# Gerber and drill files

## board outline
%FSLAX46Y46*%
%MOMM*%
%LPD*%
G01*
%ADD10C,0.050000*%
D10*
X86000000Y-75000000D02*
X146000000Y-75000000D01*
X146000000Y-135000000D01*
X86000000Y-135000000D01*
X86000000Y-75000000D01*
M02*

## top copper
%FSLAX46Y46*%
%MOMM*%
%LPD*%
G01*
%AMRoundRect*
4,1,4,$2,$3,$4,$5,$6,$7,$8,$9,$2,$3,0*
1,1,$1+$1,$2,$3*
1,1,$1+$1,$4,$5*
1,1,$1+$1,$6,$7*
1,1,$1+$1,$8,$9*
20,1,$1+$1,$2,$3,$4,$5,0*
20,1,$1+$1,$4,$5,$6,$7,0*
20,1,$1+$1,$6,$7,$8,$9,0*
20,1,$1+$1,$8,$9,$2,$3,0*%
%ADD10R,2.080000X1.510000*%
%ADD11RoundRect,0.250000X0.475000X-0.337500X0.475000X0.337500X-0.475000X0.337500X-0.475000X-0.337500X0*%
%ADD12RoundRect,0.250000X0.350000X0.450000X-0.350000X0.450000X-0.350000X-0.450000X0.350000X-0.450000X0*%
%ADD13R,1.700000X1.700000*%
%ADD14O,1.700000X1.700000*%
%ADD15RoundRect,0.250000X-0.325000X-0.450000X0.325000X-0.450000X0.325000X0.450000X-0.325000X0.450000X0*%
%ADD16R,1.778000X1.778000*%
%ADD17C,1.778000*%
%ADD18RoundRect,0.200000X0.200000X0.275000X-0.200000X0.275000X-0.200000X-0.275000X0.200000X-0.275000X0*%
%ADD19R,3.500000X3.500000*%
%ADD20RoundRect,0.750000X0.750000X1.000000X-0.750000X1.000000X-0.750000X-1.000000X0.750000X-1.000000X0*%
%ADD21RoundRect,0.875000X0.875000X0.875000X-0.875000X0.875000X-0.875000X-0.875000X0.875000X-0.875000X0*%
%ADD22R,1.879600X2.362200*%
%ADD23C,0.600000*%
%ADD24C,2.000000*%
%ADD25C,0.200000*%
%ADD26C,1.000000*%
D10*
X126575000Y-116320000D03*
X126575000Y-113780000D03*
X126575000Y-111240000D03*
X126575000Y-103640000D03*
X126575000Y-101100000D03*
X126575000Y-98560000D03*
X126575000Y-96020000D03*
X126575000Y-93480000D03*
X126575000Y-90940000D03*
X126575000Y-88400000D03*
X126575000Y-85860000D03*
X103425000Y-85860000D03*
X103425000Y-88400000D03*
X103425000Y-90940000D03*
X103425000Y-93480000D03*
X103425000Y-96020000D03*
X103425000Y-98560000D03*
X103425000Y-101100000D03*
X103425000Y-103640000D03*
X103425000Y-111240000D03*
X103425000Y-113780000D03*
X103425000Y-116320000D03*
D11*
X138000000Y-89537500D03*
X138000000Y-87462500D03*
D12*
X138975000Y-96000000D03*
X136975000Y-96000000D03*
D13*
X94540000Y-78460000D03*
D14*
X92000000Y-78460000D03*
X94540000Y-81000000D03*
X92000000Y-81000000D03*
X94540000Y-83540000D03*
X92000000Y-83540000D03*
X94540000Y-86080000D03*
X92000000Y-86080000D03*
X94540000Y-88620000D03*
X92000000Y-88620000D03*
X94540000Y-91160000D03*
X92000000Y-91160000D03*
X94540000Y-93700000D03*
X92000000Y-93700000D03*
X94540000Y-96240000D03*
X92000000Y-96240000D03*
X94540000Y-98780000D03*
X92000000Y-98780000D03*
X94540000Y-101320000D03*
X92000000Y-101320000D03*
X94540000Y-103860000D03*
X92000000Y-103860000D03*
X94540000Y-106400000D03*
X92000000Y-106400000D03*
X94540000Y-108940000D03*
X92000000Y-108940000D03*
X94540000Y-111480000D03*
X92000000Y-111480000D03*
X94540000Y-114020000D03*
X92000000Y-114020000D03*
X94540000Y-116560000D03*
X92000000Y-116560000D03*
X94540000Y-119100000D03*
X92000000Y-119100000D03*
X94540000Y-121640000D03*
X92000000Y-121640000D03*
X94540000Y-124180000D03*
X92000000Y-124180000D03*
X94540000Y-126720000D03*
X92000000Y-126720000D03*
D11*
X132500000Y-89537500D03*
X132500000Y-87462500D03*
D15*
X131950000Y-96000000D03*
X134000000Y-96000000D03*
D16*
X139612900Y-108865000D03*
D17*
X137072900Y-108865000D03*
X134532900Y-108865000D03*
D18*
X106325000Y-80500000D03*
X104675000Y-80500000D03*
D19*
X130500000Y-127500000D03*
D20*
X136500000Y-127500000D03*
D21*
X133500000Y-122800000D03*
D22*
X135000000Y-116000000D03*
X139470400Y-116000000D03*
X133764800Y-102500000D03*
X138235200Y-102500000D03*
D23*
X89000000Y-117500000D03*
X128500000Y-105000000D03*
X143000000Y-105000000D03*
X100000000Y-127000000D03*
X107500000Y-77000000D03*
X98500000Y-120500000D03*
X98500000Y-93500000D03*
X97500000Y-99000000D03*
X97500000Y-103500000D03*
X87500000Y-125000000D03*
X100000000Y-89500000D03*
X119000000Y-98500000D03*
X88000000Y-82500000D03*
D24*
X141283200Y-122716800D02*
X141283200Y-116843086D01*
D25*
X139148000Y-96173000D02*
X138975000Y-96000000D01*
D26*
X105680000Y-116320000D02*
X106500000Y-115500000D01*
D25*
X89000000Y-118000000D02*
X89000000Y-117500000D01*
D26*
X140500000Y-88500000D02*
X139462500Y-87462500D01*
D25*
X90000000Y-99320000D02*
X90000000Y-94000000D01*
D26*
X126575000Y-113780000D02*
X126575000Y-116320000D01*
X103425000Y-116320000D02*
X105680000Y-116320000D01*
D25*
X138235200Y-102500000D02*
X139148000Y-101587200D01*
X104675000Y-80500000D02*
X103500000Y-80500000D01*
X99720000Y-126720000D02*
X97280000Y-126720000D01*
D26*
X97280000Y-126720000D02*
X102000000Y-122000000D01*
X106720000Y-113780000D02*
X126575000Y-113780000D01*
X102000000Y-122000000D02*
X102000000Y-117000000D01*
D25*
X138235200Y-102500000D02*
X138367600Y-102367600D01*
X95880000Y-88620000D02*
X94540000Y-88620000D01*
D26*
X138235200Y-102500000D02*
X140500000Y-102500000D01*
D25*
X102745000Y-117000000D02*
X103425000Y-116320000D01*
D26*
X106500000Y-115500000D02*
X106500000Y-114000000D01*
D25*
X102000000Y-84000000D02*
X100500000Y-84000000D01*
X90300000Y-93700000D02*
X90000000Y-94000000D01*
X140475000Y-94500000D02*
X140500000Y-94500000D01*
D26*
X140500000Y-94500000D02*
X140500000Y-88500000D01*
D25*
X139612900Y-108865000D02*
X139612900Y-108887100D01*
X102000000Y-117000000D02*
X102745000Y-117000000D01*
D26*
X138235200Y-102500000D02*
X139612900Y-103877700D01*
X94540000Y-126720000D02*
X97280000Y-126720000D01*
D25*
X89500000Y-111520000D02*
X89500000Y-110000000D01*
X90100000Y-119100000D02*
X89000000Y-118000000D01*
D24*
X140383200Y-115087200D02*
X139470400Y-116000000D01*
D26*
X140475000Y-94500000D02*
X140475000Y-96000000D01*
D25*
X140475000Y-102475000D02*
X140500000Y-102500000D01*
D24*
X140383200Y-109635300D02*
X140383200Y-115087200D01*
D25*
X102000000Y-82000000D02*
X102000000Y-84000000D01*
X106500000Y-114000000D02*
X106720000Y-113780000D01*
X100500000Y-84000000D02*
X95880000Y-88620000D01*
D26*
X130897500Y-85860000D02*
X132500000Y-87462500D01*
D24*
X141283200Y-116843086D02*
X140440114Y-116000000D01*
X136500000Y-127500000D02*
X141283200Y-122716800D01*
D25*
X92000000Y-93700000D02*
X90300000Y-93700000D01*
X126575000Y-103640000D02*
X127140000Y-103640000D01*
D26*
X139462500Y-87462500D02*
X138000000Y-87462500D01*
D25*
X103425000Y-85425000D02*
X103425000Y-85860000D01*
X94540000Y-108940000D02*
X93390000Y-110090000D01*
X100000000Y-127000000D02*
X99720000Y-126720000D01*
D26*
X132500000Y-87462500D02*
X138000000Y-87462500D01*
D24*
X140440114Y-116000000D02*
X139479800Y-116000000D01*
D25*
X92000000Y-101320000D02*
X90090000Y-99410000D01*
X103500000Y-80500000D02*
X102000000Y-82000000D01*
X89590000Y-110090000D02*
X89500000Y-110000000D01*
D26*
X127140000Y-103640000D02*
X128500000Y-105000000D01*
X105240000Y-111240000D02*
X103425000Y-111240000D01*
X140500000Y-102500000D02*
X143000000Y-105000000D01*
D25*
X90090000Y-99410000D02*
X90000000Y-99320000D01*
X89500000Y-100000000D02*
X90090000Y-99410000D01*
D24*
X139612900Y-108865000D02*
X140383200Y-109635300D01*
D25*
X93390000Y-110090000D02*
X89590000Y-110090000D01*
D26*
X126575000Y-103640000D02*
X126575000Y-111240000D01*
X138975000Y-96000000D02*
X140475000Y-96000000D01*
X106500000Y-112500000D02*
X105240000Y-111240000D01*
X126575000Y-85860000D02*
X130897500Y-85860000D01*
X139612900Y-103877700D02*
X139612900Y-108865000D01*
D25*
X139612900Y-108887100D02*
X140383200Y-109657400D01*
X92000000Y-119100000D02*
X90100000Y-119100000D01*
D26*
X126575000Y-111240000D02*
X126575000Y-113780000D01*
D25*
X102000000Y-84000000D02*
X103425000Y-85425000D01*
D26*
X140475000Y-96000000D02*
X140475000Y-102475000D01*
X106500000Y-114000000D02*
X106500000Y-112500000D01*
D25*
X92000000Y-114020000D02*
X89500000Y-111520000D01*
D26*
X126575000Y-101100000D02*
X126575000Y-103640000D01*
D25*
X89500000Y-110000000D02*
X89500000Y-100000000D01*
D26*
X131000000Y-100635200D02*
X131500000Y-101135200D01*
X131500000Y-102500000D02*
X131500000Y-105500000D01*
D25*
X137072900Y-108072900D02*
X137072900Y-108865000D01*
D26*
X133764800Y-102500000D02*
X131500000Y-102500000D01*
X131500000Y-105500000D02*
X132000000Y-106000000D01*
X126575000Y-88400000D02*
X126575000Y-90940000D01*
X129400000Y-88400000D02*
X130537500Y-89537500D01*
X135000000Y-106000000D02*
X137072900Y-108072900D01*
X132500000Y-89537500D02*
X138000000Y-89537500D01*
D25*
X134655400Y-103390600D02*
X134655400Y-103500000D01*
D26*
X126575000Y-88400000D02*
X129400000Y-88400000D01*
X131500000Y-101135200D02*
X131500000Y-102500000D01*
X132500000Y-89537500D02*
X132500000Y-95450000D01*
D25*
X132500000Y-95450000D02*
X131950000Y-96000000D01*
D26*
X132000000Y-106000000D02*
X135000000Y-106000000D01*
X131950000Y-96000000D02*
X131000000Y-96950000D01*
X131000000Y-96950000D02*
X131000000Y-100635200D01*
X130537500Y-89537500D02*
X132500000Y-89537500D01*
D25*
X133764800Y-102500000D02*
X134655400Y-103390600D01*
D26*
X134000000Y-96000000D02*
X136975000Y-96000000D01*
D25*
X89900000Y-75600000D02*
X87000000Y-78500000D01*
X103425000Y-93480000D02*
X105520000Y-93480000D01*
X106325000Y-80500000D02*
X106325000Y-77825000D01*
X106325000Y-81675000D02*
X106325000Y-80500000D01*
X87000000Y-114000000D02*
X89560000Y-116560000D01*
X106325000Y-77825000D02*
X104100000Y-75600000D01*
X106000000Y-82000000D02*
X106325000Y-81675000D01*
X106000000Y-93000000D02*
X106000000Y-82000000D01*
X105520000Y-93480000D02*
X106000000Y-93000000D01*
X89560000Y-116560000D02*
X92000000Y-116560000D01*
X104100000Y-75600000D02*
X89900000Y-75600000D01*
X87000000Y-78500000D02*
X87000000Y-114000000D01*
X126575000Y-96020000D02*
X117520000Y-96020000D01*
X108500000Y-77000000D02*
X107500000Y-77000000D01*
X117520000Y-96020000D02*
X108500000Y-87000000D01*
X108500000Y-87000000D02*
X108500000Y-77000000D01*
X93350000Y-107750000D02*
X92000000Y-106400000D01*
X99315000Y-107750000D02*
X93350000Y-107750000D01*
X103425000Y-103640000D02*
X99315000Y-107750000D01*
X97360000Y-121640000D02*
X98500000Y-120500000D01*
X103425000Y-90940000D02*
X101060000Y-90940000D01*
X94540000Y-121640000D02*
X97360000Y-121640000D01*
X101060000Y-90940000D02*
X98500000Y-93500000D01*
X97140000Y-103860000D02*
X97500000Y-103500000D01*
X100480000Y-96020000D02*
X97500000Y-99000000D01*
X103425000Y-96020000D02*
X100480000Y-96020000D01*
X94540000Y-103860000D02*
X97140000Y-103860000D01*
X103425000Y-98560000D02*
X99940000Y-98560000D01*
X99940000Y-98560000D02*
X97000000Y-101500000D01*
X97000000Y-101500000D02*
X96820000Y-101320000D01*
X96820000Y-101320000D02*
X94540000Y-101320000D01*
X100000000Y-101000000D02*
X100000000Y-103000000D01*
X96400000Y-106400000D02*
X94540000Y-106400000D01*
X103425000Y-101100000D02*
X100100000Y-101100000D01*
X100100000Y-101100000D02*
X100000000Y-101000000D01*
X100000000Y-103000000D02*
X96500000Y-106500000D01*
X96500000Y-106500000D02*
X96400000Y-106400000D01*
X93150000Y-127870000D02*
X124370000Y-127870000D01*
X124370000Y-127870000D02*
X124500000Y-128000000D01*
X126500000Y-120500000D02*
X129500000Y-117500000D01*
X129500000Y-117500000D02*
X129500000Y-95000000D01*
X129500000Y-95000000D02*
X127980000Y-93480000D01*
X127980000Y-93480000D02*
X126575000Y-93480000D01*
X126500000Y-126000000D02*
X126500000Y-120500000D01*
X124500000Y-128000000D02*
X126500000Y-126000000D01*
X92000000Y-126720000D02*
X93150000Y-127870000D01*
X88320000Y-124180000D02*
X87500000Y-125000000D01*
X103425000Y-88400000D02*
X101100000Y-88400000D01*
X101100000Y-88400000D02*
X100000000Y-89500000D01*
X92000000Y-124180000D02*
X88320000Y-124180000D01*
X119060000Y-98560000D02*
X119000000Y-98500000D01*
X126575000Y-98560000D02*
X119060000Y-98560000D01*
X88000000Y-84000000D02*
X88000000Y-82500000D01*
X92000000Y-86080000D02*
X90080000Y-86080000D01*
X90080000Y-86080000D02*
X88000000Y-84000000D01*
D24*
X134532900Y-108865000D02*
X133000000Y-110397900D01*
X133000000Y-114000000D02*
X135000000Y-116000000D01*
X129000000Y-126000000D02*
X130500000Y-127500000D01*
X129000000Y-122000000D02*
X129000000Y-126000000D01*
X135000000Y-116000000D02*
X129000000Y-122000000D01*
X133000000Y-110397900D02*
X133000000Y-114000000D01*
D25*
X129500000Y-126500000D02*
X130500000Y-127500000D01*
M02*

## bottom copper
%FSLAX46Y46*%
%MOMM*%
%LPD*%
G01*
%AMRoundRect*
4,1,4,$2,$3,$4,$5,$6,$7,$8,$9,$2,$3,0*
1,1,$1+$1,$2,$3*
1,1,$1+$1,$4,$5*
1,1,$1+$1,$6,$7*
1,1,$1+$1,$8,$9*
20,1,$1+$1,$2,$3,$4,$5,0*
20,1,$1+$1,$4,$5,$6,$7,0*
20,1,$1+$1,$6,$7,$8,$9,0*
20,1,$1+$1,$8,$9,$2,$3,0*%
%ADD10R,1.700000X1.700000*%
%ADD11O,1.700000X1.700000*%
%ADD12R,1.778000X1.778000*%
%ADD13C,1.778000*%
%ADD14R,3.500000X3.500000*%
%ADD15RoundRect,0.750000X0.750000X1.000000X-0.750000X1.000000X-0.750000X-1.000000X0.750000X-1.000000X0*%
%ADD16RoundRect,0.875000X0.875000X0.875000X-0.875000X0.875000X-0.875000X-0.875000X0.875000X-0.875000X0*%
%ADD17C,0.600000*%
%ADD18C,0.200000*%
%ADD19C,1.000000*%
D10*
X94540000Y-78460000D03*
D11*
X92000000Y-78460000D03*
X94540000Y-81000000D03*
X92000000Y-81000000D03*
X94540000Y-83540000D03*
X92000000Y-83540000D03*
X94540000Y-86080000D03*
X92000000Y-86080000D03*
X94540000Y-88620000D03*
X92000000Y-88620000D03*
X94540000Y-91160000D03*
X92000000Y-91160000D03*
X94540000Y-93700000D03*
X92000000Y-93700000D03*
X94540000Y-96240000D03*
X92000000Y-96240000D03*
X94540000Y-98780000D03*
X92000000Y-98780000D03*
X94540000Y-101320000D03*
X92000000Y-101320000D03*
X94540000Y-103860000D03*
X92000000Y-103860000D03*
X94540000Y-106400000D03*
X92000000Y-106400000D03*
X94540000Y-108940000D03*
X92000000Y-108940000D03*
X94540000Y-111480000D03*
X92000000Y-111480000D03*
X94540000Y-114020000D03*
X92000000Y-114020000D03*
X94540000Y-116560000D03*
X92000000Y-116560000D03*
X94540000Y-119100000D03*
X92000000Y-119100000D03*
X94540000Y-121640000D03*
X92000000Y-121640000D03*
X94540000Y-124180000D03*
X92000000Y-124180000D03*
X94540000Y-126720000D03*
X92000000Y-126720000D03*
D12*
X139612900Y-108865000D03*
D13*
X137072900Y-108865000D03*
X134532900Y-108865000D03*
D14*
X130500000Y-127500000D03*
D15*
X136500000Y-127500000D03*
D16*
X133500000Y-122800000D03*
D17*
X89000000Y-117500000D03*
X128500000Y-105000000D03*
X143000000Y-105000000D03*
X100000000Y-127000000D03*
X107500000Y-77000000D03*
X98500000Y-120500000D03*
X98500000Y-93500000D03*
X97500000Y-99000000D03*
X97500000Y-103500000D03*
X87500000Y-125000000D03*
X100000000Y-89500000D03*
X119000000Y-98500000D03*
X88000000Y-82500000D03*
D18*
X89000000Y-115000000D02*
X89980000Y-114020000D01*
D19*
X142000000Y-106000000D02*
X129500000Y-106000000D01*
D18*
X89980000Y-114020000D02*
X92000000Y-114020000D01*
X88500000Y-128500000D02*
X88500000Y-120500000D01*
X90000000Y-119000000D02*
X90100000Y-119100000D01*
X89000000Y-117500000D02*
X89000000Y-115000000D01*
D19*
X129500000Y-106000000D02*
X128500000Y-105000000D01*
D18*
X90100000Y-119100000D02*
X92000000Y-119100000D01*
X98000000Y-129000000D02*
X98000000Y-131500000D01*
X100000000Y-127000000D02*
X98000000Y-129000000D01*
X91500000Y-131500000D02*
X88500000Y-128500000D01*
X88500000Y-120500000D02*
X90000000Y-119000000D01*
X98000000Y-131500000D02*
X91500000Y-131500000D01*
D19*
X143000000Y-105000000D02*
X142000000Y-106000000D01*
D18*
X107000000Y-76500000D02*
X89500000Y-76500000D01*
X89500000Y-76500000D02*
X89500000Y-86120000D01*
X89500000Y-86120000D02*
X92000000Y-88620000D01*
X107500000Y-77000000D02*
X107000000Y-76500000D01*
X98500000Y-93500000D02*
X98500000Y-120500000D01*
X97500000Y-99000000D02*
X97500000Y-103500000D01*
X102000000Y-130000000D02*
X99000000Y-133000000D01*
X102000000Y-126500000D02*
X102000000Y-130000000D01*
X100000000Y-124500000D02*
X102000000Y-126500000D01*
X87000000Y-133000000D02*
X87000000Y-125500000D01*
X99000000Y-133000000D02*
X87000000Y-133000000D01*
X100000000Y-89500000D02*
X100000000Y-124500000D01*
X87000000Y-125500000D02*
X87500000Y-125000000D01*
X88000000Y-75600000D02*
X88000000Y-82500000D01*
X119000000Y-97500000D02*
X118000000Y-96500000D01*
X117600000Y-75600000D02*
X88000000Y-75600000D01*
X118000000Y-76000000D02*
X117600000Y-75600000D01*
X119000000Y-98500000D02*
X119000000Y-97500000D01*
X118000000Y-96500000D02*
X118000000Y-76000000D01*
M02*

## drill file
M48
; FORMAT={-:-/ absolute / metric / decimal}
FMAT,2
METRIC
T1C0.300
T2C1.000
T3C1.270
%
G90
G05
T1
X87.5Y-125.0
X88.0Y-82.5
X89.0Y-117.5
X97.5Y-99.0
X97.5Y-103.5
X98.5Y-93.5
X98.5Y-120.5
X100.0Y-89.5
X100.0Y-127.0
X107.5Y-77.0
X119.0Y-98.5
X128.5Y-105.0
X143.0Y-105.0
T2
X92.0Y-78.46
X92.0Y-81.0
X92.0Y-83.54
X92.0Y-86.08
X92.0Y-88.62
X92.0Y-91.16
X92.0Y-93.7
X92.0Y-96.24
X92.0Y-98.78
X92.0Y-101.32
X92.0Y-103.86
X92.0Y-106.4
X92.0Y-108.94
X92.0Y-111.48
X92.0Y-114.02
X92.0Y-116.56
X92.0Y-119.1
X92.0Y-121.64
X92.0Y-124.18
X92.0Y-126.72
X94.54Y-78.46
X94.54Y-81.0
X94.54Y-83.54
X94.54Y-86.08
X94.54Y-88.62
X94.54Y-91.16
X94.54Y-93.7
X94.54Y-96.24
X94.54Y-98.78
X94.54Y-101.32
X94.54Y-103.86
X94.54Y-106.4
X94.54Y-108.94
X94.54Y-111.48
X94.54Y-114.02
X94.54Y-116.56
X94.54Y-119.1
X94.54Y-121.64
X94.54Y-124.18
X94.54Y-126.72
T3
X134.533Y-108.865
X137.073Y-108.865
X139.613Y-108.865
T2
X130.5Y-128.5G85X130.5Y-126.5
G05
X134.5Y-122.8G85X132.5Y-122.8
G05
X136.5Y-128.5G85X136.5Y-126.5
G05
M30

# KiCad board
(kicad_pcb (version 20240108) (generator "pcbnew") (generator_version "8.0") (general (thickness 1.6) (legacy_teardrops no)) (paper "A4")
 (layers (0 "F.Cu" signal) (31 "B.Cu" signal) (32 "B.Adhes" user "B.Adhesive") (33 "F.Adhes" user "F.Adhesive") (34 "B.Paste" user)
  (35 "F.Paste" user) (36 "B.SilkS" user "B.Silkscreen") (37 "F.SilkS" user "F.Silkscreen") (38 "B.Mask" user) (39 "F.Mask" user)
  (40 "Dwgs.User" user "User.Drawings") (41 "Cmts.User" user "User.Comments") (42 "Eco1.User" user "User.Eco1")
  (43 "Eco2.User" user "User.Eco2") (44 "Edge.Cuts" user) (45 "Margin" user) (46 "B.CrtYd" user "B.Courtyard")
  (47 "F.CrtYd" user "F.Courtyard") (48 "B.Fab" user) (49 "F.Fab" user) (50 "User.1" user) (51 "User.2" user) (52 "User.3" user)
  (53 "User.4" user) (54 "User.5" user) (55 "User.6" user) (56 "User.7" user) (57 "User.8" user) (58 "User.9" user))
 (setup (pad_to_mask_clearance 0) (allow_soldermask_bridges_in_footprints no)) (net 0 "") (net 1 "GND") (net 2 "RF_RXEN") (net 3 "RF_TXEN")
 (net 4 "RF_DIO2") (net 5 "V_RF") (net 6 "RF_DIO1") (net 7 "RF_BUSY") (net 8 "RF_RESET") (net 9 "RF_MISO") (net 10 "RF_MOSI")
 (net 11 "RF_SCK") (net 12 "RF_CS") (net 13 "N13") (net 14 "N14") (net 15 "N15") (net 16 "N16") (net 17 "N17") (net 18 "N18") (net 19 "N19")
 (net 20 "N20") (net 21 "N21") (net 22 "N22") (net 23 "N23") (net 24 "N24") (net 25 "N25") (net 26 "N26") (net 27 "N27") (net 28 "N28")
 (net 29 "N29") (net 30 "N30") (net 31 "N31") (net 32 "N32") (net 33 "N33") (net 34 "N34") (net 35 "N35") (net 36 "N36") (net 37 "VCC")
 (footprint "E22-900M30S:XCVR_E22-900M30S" (layer "F.Cu") (at 115 102.5)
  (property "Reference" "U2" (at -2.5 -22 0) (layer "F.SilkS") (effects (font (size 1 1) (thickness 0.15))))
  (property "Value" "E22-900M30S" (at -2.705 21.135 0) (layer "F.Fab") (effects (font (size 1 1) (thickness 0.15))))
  (pad "1" smd rect (at 11.575 13.82) (size 2.08 1.51) (layers "F.Cu" "F.Paste" "F.Mask") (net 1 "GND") (solder_mask_margin 0.102))
  (pad "2" smd rect (at 11.575 11.28) (size 2.08 1.51) (layers "F.Cu" "F.Paste" "F.Mask") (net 1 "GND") (solder_mask_margin 0.102))
  (pad "3" smd rect (at 11.575 8.74) (size 2.08 1.51) (layers "F.Cu" "F.Paste" "F.Mask") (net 1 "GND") (solder_mask_margin 0.102))
  (pad "4" smd rect (at 11.575 1.14) (size 2.08 1.51) (layers "F.Cu" "F.Paste" "F.Mask") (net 1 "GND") (solder_mask_margin 0.102))
  (pad "5" smd rect (at 11.575 -1.4) (size 2.08 1.51) (layers "F.Cu" "F.Paste" "F.Mask") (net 1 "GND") (solder_mask_margin 0.102))
  (pad "6" smd rect (at 11.575 -3.94) (size 2.08 1.51) (layers "F.Cu" "F.Paste" "F.Mask") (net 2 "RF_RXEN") (solder_mask_margin 0.102))
  (pad "7" smd rect (at 11.575 -6.48) (size 2.08 1.51) (layers "F.Cu" "F.Paste" "F.Mask") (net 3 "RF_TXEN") (solder_mask_margin 0.102))
  (pad "8" smd rect (at 11.575 -9.02) (size 2.08 1.51) (layers "F.Cu" "F.Paste" "F.Mask") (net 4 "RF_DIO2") (solder_mask_margin 0.102))
  (pad "9" smd rect (at 11.575 -11.56) (size 2.08 1.51) (layers "F.Cu" "F.Paste" "F.Mask") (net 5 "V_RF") (solder_mask_margin 0.102))
  (pad "10" smd rect (at 11.575 -14.1) (size 2.08 1.51) (layers "F.Cu" "F.Paste" "F.Mask") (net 5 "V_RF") (solder_mask_margin 0.102))
  (pad "11" smd rect (at 11.575 -16.64) (size 2.08 1.51) (layers "F.Cu" "F.Paste" "F.Mask") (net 1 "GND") (solder_mask_margin 0.102))
  (pad "12" smd rect (at -11.575 -16.64) (size 2.08 1.51) (layers "F.Cu" "F.Paste" "F.Mask") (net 1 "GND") (solder_mask_margin 0.102))
  (pad "13" smd rect (at -11.575 -14.1) (size 2.08 1.51) (layers "F.Cu" "F.Paste" "F.Mask") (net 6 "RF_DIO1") (solder_mask_margin 0.102))
  (pad "14" smd rect (at -11.575 -11.56) (size 2.08 1.51) (layers "F.Cu" "F.Paste" "F.Mask") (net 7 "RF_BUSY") (solder_mask_margin 0.102))
  (pad "15" smd rect (at -11.575 -9.02) (size 2.08 1.51) (layers "F.Cu" "F.Paste" "F.Mask") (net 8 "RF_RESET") (solder_mask_margin 0.102))
  (pad "16" smd rect (at -11.575 -6.48) (size 2.08 1.51) (layers "F.Cu" "F.Paste" "F.Mask") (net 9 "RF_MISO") (solder_mask_margin 0.102))
  (pad "17" smd rect (at -11.575 -3.94) (size 2.08 1.51) (layers "F.Cu" "F.Paste" "F.Mask") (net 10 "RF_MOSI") (solder_mask_margin 0.102))
  (pad "18" smd rect (at -11.575 -1.4) (size 2.08 1.51) (layers "F.Cu" "F.Paste" "F.Mask") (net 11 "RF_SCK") (solder_mask_margin 0.102))
  (pad "19" smd rect (at -11.575 1.14) (size 2.08 1.51) (layers "F.Cu" "F.Paste" "F.Mask") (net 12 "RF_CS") (solder_mask_margin 0.102))
  (pad "20" smd rect (at -11.575 8.74) (size 2.08 1.51) (layers "F.Cu" "F.Paste" "F.Mask") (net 1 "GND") (solder_mask_margin 0.102))
  (pad "21" smd rect (at -11.575 11.28) (size 2.08 1.51) (layers "F.Cu" "F.Paste" "F.Mask") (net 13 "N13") (solder_mask_margin 0.102))
  (pad "22" smd rect (at -11.575 13.82) (size 2.08 1.51) (layers "F.Cu" "F.Paste" "F.Mask") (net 1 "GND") (solder_mask_margin 0.102)))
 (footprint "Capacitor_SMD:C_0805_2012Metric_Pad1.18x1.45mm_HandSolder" (layer "F.Cu") (at 138 88.5 90)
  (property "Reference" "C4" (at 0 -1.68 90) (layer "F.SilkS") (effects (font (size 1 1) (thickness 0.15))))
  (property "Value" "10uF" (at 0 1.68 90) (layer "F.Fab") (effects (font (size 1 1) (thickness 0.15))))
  (pad "1" smd roundrect (at -1.0375 0 90) (size 1.175 1.45) (layers "F.Cu" "F.Paste" "F.Mask") (roundrect_rratio 0.212766) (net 5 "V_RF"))
  (pad "2" smd roundrect (at 1.0375 0 90) (size 1.175 1.45) (layers "F.Cu" "F.Paste" "F.Mask") (roundrect_rratio 0.212766) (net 1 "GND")))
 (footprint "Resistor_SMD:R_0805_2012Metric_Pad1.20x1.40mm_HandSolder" (layer "F.Cu") (at 137.975 96 180)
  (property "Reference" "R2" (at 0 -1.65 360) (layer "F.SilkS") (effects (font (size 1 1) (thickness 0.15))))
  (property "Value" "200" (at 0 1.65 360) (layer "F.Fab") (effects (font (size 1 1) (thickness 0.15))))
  (pad "1" smd roundrect (at -1 0 180) (size 1.2 1.4) (layers "F.Cu" "F.Paste" "F.Mask") (roundrect_rratio 0.208333) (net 1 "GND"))
  (pad "2" smd roundrect (at 1 0 180) (size 1.2 1.4) (layers "F.Cu" "F.Paste" "F.Mask") (roundrect_rratio 0.208333) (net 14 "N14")))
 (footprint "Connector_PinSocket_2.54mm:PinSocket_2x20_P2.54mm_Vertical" (layer "F.Cu") (at 94.54 78.46)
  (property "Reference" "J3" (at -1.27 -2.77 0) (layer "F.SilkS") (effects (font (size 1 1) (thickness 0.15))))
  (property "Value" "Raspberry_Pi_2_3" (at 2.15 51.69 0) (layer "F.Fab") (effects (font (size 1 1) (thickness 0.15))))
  (pad "1" thru_hole rect (at 0 0) (size 1.7 1.7) (drill 1) (layers "*.Cu" "*.Mask") (remove_unused_layers no) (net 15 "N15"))
  (pad "2" thru_hole oval (at -2.54 0) (size 1.7 1.7) (drill 1) (layers "*.Cu" "*.Mask") (remove_unused_layers no) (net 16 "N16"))
  (pad "3" thru_hole oval (at 0 2.54) (size 1.7 1.7) (drill 1) (layers "*.Cu" "*.Mask") (remove_unused_layers no) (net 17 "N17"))
  (pad "4" thru_hole oval (at -2.54 2.54) (size 1.7 1.7) (drill 1) (layers "*.Cu" "*.Mask") (remove_unused_layers no) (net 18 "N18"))
  (pad "5" thru_hole oval (at 0 5.08) (size 1.7 1.7) (drill 1) (layers "*.Cu" "*.Mask") (remove_unused_layers no) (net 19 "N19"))
  (pad "6" thru_hole oval (at -2.54 5.08) (size 1.7 1.7) (drill 1) (layers "*.Cu" "*.Mask") (remove_unused_layers no) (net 1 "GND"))
  (pad "7" thru_hole oval (at 0 7.62) (size 1.7 1.7) (drill 1) (layers "*.Cu" "*.Mask") (remove_unused_layers no) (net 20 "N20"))
  (pad "8" thru_hole oval (at -2.54 7.62) (size 1.7 1.7) (drill 1) (layers "*.Cu" "*.Mask") (remove_unused_layers no) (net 2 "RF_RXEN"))
  (pad "9" thru_hole oval (at 0 10.16) (size 1.7 1.7) (drill 1) (layers "*.Cu" "*.Mask") (remove_unused_layers no) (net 1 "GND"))
  (pad "10" thru_hole oval (at -2.54 10.16) (size 1.7 1.7) (drill 1) (layers "*.Cu" "*.Mask") (remove_unused_layers no) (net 3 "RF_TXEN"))
  (pad "11" thru_hole oval (at 0 12.7) (size 1.7 1.7) (drill 1) (layers "*.Cu" "*.Mask") (remove_unused_layers no) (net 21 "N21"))
  (pad "12" thru_hole oval (at -2.54 12.7) (size 1.7 1.7) (drill 1) (layers "*.Cu" "*.Mask") (remove_unused_layers no) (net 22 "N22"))
  (pad "13" thru_hole oval (at 0 15.24) (size 1.7 1.7) (drill 1) (layers "*.Cu" "*.Mask") (remove_unused_layers no) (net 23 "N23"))
  (pad "14" thru_hole oval (at -2.54 15.24) (size 1.7 1.7) (drill 1) (layers "*.Cu" "*.Mask") (remove_unused_layers no) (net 1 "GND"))
  (pad "15" thru_hole oval (at 0 17.78) (size 1.7 1.7) (drill 1) (layers "*.Cu" "*.Mask") (remove_unused_layers no) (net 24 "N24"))
  (pad "16" thru_hole oval (at -2.54 17.78) (size 1.7 1.7) (drill 1) (layers "*.Cu" "*.Mask") (remove_unused_layers no) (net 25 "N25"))
  (pad "17" thru_hole oval (at 0 20.32) (size 1.7 1.7) (drill 1) (layers "*.Cu" "*.Mask") (remove_unused_layers no) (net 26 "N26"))
  (pad "18" thru_hole oval (at -2.54 20.32) (size 1.7 1.7) (drill 1) (layers "*.Cu" "*.Mask") (remove_unused_layers no) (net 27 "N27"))
  (pad "19" thru_hole oval (at 0 22.86) (size 1.7 1.7) (drill 1) (layers "*.Cu" "*.Mask") (remove_unused_layers no) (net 10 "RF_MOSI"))
  (pad "20" thru_hole oval (at -2.54 22.86) (size 1.7 1.7) (drill 1) (layers "*.Cu" "*.Mask") (remove_unused_layers no) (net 1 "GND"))
  (pad "21" thru_hole oval (at 0 25.4) (size 1.7 1.7) (drill 1) (layers "*.Cu" "*.Mask") (remove_unused_layers no) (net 9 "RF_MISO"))
  (pad "22" thru_hole oval (at -2.54 25.4) (size 1.7 1.7) (drill 1) (layers "*.Cu" "*.Mask") (remove_unused_layers no) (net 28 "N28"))
  (pad "23" thru_hole oval (at 0 27.94) (size 1.7 1.7) (drill 1) (layers "*.Cu" "*.Mask") (remove_unused_layers no) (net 11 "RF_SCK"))
  (pad "24" thru_hole oval (at -2.54 27.94) (size 1.7 1.7) (drill 1) (layers "*.Cu" "*.Mask") (remove_unused_layers no) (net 12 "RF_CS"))
  (pad "25" thru_hole oval (at 0 30.48) (size 1.7 1.7) (drill 1) (layers "*.Cu" "*.Mask") (remove_unused_layers no) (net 1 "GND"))
  (pad "26" thru_hole oval (at -2.54 30.48) (size 1.7 1.7) (drill 1) (layers "*.Cu" "*.Mask") (remove_unused_layers no) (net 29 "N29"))
  (pad "27" thru_hole oval (at 0 33.02) (size 1.7 1.7) (drill 1) (layers "*.Cu" "*.Mask") (remove_unused_layers no) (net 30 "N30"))
  (pad "28" thru_hole oval (at -2.54 33.02) (size 1.7 1.7) (drill 1) (layers "*.Cu" "*.Mask") (remove_unused_layers no) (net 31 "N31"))
  (pad "29" thru_hole oval (at 0 35.56) (size 1.7 1.7) (drill 1) (layers "*.Cu" "*.Mask") (remove_unused_layers no) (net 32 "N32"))
  (pad "30" thru_hole oval (at -2.54 35.56) (size 1.7 1.7) (drill 1) (layers "*.Cu" "*.Mask") (remove_unused_layers no) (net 1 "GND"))
  (pad "31" thru_hole oval (at 0 38.1) (size 1.7 1.7) (drill 1) (layers "*.Cu" "*.Mask") (remove_unused_layers no) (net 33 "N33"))
  (pad "32" thru_hole oval (at -2.54 38.1) (size 1.7 1.7) (drill 1) (layers "*.Cu" "*.Mask") (remove_unused_layers no) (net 8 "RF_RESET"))
  (pad "33" thru_hole oval (at 0 40.64) (size 1.7 1.7) (drill 1) (layers "*.Cu" "*.Mask") (remove_unused_layers no) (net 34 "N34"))
  (pad "34" thru_hole oval (at -2.54 40.64) (size 1.7 1.7) (drill 1) (layers "*.Cu" "*.Mask") (remove_unused_layers no) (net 1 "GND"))
  (pad "35" thru_hole oval (at 0 43.18) (size 1.7 1.7) (drill 1) (layers "*.Cu" "*.Mask") (remove_unused_layers no) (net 7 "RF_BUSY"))
  (pad "36" thru_hole oval (at -2.54 43.18) (size 1.7 1.7) (drill 1) (layers "*.Cu" "*.Mask") (remove_unused_layers no) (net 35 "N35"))
  (pad "37" thru_hole oval (at 0 45.72) (size 1.7 1.7) (drill 1) (layers "*.Cu" "*.Mask") (remove_unused_layers no) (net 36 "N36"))
  (pad "38" thru_hole oval (at -2.54 45.72) (size 1.7 1.7) (drill 1) (layers "*.Cu" "*.Mask") (remove_unused_layers no) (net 6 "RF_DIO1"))
  (pad "39" thru_hole oval (at 0 48.26) (size 1.7 1.7) (drill 1) (layers "*.Cu" "*.Mask") (remove_unused_layers no) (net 1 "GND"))
  (pad "40" thru_hole oval (at -2.54 48.26) (size 1.7 1.7) (drill 1) (layers "*.Cu" "*.Mask") (remove_unused_layers no) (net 4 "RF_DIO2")))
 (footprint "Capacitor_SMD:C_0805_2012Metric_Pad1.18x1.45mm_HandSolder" (layer "F.Cu") (at 132.5 88.5 90)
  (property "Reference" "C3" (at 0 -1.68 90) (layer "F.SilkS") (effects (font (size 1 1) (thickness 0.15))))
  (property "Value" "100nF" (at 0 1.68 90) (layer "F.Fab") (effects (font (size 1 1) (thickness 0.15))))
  (pad "1" smd roundrect (at -1.0375 0 90) (size 1.175 1.45) (layers "F.Cu" "F.Paste" "F.Mask") (roundrect_rratio 0.212766) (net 5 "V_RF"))
  (pad "2" smd roundrect (at 1.0375 0 90) (size 1.175 1.45) (layers "F.Cu" "F.Paste" "F.Mask") (roundrect_rratio 0.212766) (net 1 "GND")))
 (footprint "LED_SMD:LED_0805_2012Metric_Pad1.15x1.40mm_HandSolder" (layer "F.Cu") (at 132.975 96)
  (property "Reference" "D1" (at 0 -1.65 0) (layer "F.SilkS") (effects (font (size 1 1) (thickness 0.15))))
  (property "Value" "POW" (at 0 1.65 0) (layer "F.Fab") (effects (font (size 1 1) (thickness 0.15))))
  (pad "1" smd roundrect (at -1.025 0) (size 1.15 1.4) (layers "F.Cu" "F.Paste" "F.Mask") (roundrect_rratio 0.217391) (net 5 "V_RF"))
  (pad "2" smd roundrect (at 1.025 0) (size 1.15 1.4) (layers "F.Cu" "F.Paste" "F.Mask") (roundrect_rratio 0.217391) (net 14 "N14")))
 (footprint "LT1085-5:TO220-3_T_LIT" (layer "F.Cu") (at 139.6129 108.865 180)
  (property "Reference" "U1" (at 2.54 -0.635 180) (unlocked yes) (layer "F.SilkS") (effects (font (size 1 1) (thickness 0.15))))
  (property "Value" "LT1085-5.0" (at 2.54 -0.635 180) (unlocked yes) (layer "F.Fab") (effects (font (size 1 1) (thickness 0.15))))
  (pad "1" thru_hole rect (at 0 0 180) (size 1.778 1.778) (drill 1.27) (layers "*.Cu" "*.Mask") (remove_unused_layers no) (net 1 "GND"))
  (pad "2" thru_hole circle (at 2.54 0 180) (size 1.778 1.778) (drill 1.27) (layers "*.Cu" "*.Mask") (remove_unused_layers no)
   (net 5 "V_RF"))
  (pad "3" thru_hole circle (at 5.08 0 180) (size 1.778 1.778) (drill 1.27) (layers "*.Cu" "*.Mask") (remove_unused_layers no)
   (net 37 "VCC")))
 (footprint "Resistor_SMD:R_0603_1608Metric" (layer "F.Cu") (at 105.5 80.5 180)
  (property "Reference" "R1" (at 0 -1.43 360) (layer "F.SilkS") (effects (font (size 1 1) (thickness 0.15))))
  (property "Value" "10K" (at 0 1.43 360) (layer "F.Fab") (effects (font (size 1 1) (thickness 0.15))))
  (pad "1" smd roundrect (at -0.825 0 180) (size 0.8 0.95) (layers "F.Cu" "F.Paste" "F.Mask") (roundrect_rratio 0.25) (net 8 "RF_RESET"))
  (pad "2" smd roundrect (at 0.825 0 180) (size 0.8 0.95) (layers "F.Cu" "F.Paste" "F.Mask") (roundrect_rratio 0.25) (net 1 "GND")))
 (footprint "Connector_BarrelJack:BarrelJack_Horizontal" (layer "F.Cu") (at 130.5 127.5 180)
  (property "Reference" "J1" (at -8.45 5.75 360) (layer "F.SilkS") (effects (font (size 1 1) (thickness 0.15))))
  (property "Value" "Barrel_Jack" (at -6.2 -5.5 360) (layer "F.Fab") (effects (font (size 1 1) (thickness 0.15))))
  (pad "1" thru_hole rect (at 0 0 180) (size 3.5 3.5) (drill oval 1 3) (layers "*.Cu" "*.Mask") (remove_unused_layers no) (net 37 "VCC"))
  (pad "2" thru_hole roundrect (at -6 0 180) (size 3 3.5) (drill oval 1 3) (layers "*.Cu" "*.Mask") (remove_unused_layers no)
   (roundrect_rratio 0.25) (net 1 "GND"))
  (pad "3" thru_hole roundrect (at -3 4.7 180) (size 3.5 3.5) (drill oval 3 1) (layers "*.Cu" "*.Mask") (remove_unused_layers no)
   (roundrect_rratio 0.25)))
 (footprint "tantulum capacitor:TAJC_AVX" (layer "F.Cu") (at 137.2352 116)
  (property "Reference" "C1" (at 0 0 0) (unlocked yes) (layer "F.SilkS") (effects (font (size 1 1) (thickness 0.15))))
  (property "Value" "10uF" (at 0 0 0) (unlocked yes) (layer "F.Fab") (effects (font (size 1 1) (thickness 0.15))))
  (pad "1" smd rect (at -2.2352 0 90) (size 2.3622 1.8796) (layers "F.Cu" "F.Paste" "F.Mask") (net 37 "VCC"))
  (pad "2" smd rect (at 2.2352 0 90) (size 2.3622 1.8796) (layers "F.Cu" "F.Paste" "F.Mask") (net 1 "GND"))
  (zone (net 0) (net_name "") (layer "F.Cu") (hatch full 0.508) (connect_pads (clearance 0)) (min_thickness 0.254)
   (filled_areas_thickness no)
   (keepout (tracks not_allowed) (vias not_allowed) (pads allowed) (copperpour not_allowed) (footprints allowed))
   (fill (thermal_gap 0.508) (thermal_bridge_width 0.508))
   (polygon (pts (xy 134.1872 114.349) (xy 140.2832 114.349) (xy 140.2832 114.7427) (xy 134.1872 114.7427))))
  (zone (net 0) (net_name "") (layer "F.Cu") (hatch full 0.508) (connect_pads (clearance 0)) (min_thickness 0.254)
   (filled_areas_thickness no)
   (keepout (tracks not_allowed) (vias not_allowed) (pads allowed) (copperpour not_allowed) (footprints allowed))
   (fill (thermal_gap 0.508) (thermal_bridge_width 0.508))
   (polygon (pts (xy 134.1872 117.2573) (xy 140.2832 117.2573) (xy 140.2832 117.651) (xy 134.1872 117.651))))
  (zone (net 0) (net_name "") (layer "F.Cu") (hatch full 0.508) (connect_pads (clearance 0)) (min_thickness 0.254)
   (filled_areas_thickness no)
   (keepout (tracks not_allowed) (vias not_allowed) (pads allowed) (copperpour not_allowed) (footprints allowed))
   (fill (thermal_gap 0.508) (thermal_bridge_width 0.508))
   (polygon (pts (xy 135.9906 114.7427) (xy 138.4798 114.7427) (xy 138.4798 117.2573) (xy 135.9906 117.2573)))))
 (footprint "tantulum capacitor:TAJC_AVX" (layer "F.Cu") (at 136 102.5)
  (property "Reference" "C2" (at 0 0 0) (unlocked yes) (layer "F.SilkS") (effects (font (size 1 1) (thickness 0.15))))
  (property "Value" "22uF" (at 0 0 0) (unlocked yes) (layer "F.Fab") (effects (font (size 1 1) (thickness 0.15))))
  (pad "1" smd rect (at -2.2352 0 90) (size 2.3622 1.8796) (layers "F.Cu" "F.Paste" "F.Mask") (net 5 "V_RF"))
  (pad "2" smd rect (at 2.2352 0 90) (size 2.3622 1.8796) (layers "F.Cu" "F.Paste" "F.Mask") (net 1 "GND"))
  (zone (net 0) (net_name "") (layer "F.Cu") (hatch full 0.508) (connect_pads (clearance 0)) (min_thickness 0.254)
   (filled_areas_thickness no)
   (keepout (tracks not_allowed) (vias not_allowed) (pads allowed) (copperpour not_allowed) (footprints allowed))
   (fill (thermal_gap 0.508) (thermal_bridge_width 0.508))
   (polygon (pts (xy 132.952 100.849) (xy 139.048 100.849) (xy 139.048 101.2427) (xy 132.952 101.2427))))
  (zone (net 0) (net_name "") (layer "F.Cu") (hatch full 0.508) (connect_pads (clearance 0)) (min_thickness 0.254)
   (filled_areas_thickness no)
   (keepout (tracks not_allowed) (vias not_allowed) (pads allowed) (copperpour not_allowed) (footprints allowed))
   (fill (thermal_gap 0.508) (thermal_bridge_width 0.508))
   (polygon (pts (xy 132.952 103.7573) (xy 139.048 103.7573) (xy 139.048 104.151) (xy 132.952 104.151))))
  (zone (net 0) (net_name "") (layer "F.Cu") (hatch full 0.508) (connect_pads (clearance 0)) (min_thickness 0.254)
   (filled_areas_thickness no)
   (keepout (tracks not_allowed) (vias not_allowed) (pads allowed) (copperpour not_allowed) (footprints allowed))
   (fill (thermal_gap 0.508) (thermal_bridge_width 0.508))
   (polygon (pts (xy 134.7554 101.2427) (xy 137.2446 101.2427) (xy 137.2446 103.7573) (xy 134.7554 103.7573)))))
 (gr_rect (start 86 75) (end 146 135) (stroke (width 0.05) (type default)) (fill none) (layer "Edge.Cuts"))
 (segment (start 141.2832 122.7168) (end 141.2832 116.843086) (width 2) (layer "F.Cu") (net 1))
 (segment (start 139.148 96.173) (end 138.975 96) (width 0.2) (layer "F.Cu") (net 1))
 (segment (start 105.68 116.32) (end 106.5 115.5) (width 1) (layer "F.Cu") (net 1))
 (segment (start 89 118) (end 89 117.5) (width 0.2) (layer "F.Cu") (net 1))
 (segment (start 140.5 88.5) (end 139.4625 87.4625) (width 1) (layer "F.Cu") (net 1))
 (segment (start 90 99.32) (end 90 94) (width 0.2) (layer "F.Cu") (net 1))
 (segment (start 126.575 113.78) (end 126.575 116.32) (width 1) (layer "F.Cu") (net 1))
 (segment (start 103.425 116.32) (end 105.68 116.32) (width 1) (layer "F.Cu") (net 1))
 (segment (start 138.2352 102.5) (end 139.148 101.5872) (width 0.2) (layer "F.Cu") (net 1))
 (segment (start 104.675 80.5) (end 103.5 80.5) (width 0.2) (layer "F.Cu") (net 1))
 (segment (start 99.72 126.72) (end 97.28 126.72) (width 0.2) (layer "F.Cu") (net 1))
 (segment (start 97.28 126.72) (end 102 122) (width 1) (layer "F.Cu") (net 1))
 (segment (start 106.72 113.78) (end 126.575 113.78) (width 1) (layer "F.Cu") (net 1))
 (segment (start 102 122) (end 102 117) (width 1) (layer "F.Cu") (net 1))
 (segment (start 138.2352 102.5) (end 138.3676 102.3676) (width 0.2) (layer "F.Cu") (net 1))
 (segment (start 95.88 88.62) (end 94.54 88.62) (width 0.2) (layer "F.Cu") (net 1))
 (segment (start 138.2352 102.5) (end 140.5 102.5) (width 1) (layer "F.Cu") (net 1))
 (segment (start 102.745 117) (end 103.425 116.32) (width 0.2) (layer "F.Cu") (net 1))
 (segment (start 106.5 115.5) (end 106.5 114) (width 1) (layer "F.Cu") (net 1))
 (segment (start 102 84) (end 100.5 84) (width 0.2) (layer "F.Cu") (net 1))
 (segment (start 90.3 93.7) (end 90 94) (width 0.2) (layer "F.Cu") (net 1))
 (segment (start 140.475 94.5) (end 140.5 94.5) (width 0.2) (layer "F.Cu") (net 1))
 (segment (start 140.5 94.5) (end 140.5 88.5) (width 1) (layer "F.Cu") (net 1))
 (segment (start 139.6129 108.865) (end 139.6129 108.8871) (width 0.2) (layer "F.Cu") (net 1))
 (segment (start 102 117) (end 102.745 117) (width 0.2) (layer "F.Cu") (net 1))
 (segment (start 138.2352 102.5) (end 139.6129 103.8777) (width 1) (layer "F.Cu") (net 1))
 (segment (start 94.54 126.72) (end 97.28 126.72) (width 1) (layer "F.Cu") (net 1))
 (segment (start 89.5 111.52) (end 89.5 110) (width 0.2) (layer "F.Cu") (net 1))
 (segment (start 90.1 119.1) (end 89 118) (width 0.2) (layer "F.Cu") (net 1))
 (segment (start 140.3832 115.0872) (end 139.4704 116) (width 2) (layer "F.Cu") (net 1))
 (segment (start 140.475 94.5) (end 140.475 96) (width 1) (layer "F.Cu") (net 1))
 (segment (start 140.475 102.475) (end 140.5 102.5) (width 0.2) (layer "F.Cu") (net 1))
 (segment (start 140.3832 109.6353) (end 140.3832 115.0872) (width 2) (layer "F.Cu") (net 1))
 (segment (start 102 82) (end 102 84) (width 0.2) (layer "F.Cu") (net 1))
 (segment (start 106.5 114) (end 106.72 113.78) (width 0.2) (layer "F.Cu") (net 1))
 (segment (start 100.5 84) (end 95.88 88.62) (width 0.2) (layer "F.Cu") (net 1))
 (segment (start 130.8975 85.86) (end 132.5 87.4625) (width 1) (layer "F.Cu") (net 1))
 (segment (start 141.2832 116.843086) (end 140.440114 116) (width 2) (layer "F.Cu") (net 1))
 (segment (start 136.5 127.5) (end 141.2832 122.7168) (width 2) (layer "F.Cu") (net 1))
 (segment (start 92 93.7) (end 90.3 93.7) (width 0.2) (layer "F.Cu") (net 1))
 (segment (start 126.575 103.64) (end 127.14 103.64) (width 0.2) (layer "F.Cu") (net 1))
 (segment (start 139.4625 87.4625) (end 138 87.4625) (width 1) (layer "F.Cu") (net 1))
 (segment (start 103.425 85.425) (end 103.425 85.86) (width 0.2) (layer "F.Cu") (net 1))
 (segment (start 94.54 108.94) (end 93.39 110.09) (width 0.2) (layer "F.Cu") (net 1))
 (segment (start 100 127) (end 99.72 126.72) (width 0.2) (layer "F.Cu") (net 1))
 (segment (start 132.5 87.4625) (end 138 87.4625) (width 1) (layer "F.Cu") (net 1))
 (segment (start 140.440114 116) (end 139.4798 116) (width 2) (layer "F.Cu") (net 1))
 (segment (start 92 101.32) (end 90.09 99.41) (width 0.2) (layer "F.Cu") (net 1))
 (segment (start 103.5 80.5) (end 102 82) (width 0.2) (layer "F.Cu") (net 1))
 (segment (start 89.59 110.09) (end 89.5 110) (width 0.2) (layer "F.Cu") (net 1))
 (segment (start 127.14 103.64) (end 128.5 105) (width 1) (layer "F.Cu") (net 1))
 (segment (start 105.24 111.24) (end 103.425 111.24) (width 1) (layer "F.Cu") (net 1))
 (segment (start 140.5 102.5) (end 143 105) (width 1) (layer "F.Cu") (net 1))
 (segment (start 90.09 99.41) (end 90 99.32) (width 0.2) (layer "F.Cu") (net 1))
 (segment (start 89.5 100) (end 90.09 99.41) (width 0.2) (layer "F.Cu") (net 1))
 (segment (start 139.6129 108.865) (end 140.3832 109.6353) (width 2) (layer "F.Cu") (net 1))
 (segment (start 93.39 110.09) (end 89.59 110.09) (width 0.2) (layer "F.Cu") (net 1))
 (segment (start 126.575 103.64) (end 126.575 111.24) (width 1) (layer "F.Cu") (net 1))
 (segment (start 138.975 96) (end 140.475 96) (width 1) (layer "F.Cu") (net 1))
 (segment (start 106.5 112.5) (end 105.24 111.24) (width 1) (layer "F.Cu") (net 1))
 (segment (start 126.575 85.86) (end 130.8975 85.86) (width 1) (layer "F.Cu") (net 1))
 (segment (start 139.6129 103.8777) (end 139.6129 108.865) (width 1) (layer "F.Cu") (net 1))
 (segment (start 139.6129 108.8871) (end 140.3832 109.6574) (width 0.2) (layer "F.Cu") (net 1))
 (segment (start 92 119.1) (end 90.1 119.1) (width 0.2) (layer "F.Cu") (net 1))
 (segment (start 126.575 111.24) (end 126.575 113.78) (width 1) (layer "F.Cu") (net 1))
 (segment (start 102 84) (end 103.425 85.425) (width 0.2) (layer "F.Cu") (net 1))
 (segment (start 140.475 96) (end 140.475 102.475) (width 1) (layer "F.Cu") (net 1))
 (segment (start 106.5 114) (end 106.5 112.5) (width 1) (layer "F.Cu") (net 1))
 (segment (start 92 114.02) (end 89.5 111.52) (width 0.2) (layer "F.Cu") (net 1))
 (segment (start 126.575 101.1) (end 126.575 103.64) (width 1) (layer "F.Cu") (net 1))
 (segment (start 89.5 110) (end 89.5 100) (width 0.2) (layer "F.Cu") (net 1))
 (via (at 89 117.5) (size 0.6) (drill 0.3) (layers "F.Cu" "B.Cu") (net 1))
 (via (at 128.5 105) (size 0.6) (drill 0.3) (layers "F.Cu" "B.Cu") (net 1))
 (via (at 143 105) (size 0.6) (drill 0.3) (layers "F.Cu" "B.Cu") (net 1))
 (via (at 100 127) (size 0.6) (drill 0.3) (layers "F.Cu" "B.Cu") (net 1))
 (segment (start 89 115) (end 89.98 114.02) (width 0.2) (layer "B.Cu") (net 1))
 (segment (start 142 106) (end 129.5 106) (width 1) (layer "B.Cu") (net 1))
 (segment (start 89.98 114.02) (end 92 114.02) (width 0.2) (layer "B.Cu") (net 1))
 (segment (start 88.5 128.5) (end 88.5 120.5) (width 0.2) (layer "B.Cu") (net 1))
 (segment (start 90 119) (end 90.1 119.1) (width 0.2) (layer "B.Cu") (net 1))
 (segment (start 89 117.5) (end 89 115) (width 0.2) (layer "B.Cu") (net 1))
 (segment (start 129.5 106) (end 128.5 105) (width 1) (layer "B.Cu") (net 1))
 (segment (start 90.1 119.1) (end 92 119.1) (width 0.2) (layer "B.Cu") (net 1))
 (segment (start 98 129) (end 98 131.5) (width 0.2) (layer "B.Cu") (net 1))
 (segment (start 100 127) (end 98 129) (width 0.2) (layer "B.Cu") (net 1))
 (segment (start 91.5 131.5) (end 88.5 128.5) (width 0.2) (layer "B.Cu") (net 1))
 (segment (start 88.5 120.5) (end 90 119) (width 0.2) (layer "B.Cu") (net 1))
 (segment (start 98 131.5) (end 91.5 131.5) (width 0.2) (layer "B.Cu") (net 1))
 (segment (start 143 105) (end 142 106) (width 1) (layer "B.Cu") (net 1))
 (segment (start 131 100.6352) (end 131.5 101.1352) (width 1) (layer "F.Cu") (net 5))
 (segment (start 131.5 102.5) (end 131.5 105.5) (width 1) (layer "F.Cu") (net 5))
 (segment (start 137.0729 108.0729) (end 137.0729 108.865) (width 0.2) (layer "F.Cu") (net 5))
 (segment (start 133.7648 102.5) (end 131.5 102.5) (width 1) (layer "F.Cu") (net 5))
 (segment (start 131.5 105.5) (end 132 106) (width 1) (layer "F.Cu") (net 5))
 (segment (start 126.575 88.4) (end 126.575 90.94) (width 1) (layer "F.Cu") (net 5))
 (segment (start 129.4 88.4) (end 130.5375 89.5375) (width 1) (layer "F.Cu") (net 5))
 (segment (start 135 106) (end 137.0729 108.0729) (width 1) (layer "F.Cu") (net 5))
 (segment (start 132.5 89.5375) (end 138 89.5375) (width 1) (layer "F.Cu") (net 5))
 (segment (start 134.6554 103.3906) (end 134.6554 103.5) (width 0.2) (layer "F.Cu") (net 5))
 (segment (start 126.575 88.4) (end 129.4 88.4) (width 1) (layer "F.Cu") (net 5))
 (segment (start 131.5 101.1352) (end 131.5 102.5) (width 1) (layer "F.Cu") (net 5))
 (segment (start 132.5 89.5375) (end 132.5 95.45) (width 1) (layer "F.Cu") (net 5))
 (segment (start 132.5 95.45) (end 131.95 96) (width 0.2) (layer "F.Cu") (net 5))
 (segment (start 132 106) (end 135 106) (width 1) (layer "F.Cu") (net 5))
 (segment (start 131.95 96) (end 131 96.95) (width 1) (layer "F.Cu") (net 5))
 (segment (start 131 96.95) (end 131 100.6352) (width 1) (layer "F.Cu") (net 5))
 (segment (start 130.5375 89.5375) (end 132.5 89.5375) (width 1) (layer "F.Cu") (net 5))
 (segment (start 133.7648 102.5) (end 134.6554 103.3906) (width 0.2) (layer "F.Cu") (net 5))
 (segment (start 134 96) (end 136.975 96) (width 1) (layer "F.Cu") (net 14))
 (segment (start 89.9 75.6) (end 87 78.5) (width 0.2) (layer "F.Cu") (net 8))
 (segment (start 103.425 93.48) (end 105.52 93.48) (width 0.2) (layer "F.Cu") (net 8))
 (segment (start 106.325 80.5) (end 106.325 77.825) (width 0.2) (layer "F.Cu") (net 8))
 (segment (start 106.325 81.675) (end 106.325 80.5) (width 0.2) (layer "F.Cu") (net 8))
 (segment (start 87 114) (end 89.56 116.56) (width 0.2) (layer "F.Cu") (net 8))
 (segment (start 106.325 77.825) (end 104.1 75.6) (width 0.2) (layer "F.Cu") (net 8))
 (segment (start 106 82) (end 106.325 81.675) (width 0.2) (layer "F.Cu") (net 8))
 (segment (start 106 93) (end 106 82) (width 0.2) (layer "F.Cu") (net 8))
 (segment (start 105.52 93.48) (end 106 93) (width 0.2) (layer "F.Cu") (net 8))
 (segment (start 89.56 116.56) (end 92 116.56) (width 0.2) (layer "F.Cu") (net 8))
 (segment (start 104.1 75.6) (end 89.9 75.6) (width 0.2) (layer "F.Cu") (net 8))
 (segment (start 87 78.5) (end 87 114) (width 0.2) (layer "F.Cu") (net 8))
 (segment (start 126.575 96.02) (end 117.52 96.02) (width 0.2) (layer "F.Cu") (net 3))
 (segment (start 108.5 77) (end 107.5 77) (width 0.2) (layer "F.Cu") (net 3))
 (segment (start 117.52 96.02) (end 108.5 87) (width 0.2) (layer "F.Cu") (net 3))
 (segment (start 108.5 87) (end 108.5 77) (width 0.2) (layer "F.Cu") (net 3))
 (via (at 107.5 77) (size 0.6) (drill 0.3) (layers "F.Cu" "B.Cu") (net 3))
 (segment (start 107 76.5) (end 89.5 76.5) (width 0.2) (layer "B.Cu") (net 3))
 (segment (start 89.5 76.5) (end 89.5 86.12) (width 0.2) (layer "B.Cu") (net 3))
 (segment (start 89.5 86.12) (end 92 88.62) (width 0.2) (layer "B.Cu") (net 3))
 (segment (start 107.5 77) (end 107 76.5) (width 0.2) (layer "B.Cu") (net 3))
 (segment (start 93.35 107.75) (end 92 106.4) (width 0.2) (layer "F.Cu") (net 12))
 (segment (start 99.315 107.75) (end 93.35 107.75) (width 0.2) (layer "F.Cu") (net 12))
 (segment (start 103.425 103.64) (end 99.315 107.75) (width 0.2) (layer "F.Cu") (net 12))
 (segment (start 97.36 121.64) (end 98.5 120.5) (width 0.2) (layer "F.Cu") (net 7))
 (segment (start 103.425 90.94) (end 101.06 90.94) (width 0.2) (layer "F.Cu") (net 7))
 (segment (start 94.54 121.64) (end 97.36 121.64) (width 0.2) (layer "F.Cu") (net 7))
 (segment (start 101.06 90.94) (end 98.5 93.5) (width 0.2) (layer "F.Cu") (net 7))
 (via (at 98.5 120.5) (size 0.6) (drill 0.3) (layers "F.Cu" "B.Cu") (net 7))
 (via (at 98.5 93.5) (size 0.6) (drill 0.3) (layers "F.Cu" "B.Cu") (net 7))
 (segment (start 98.5 93.5) (end 98.5 120.5) (width 0.2) (layer "B.Cu") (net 7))
 (segment (start 97.14 103.86) (end 97.5 103.5) (width 0.2) (layer "F.Cu") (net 9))
 (segment (start 100.48 96.02) (end 97.5 99) (width 0.2) (layer "F.Cu") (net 9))
 (segment (start 103.425 96.02) (end 100.48 96.02) (width 0.2) (layer "F.Cu") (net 9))
 (segment (start 94.54 103.86) (end 97.14 103.86) (width 0.2) (layer "F.Cu") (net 9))
 (via (at 97.5 99) (size 0.6) (drill 0.3) (layers "F.Cu" "B.Cu") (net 9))
 (via (at 97.5 103.5) (size 0.6) (drill 0.3) (layers "F.Cu" "B.Cu") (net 9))
 (segment (start 97.5 99) (end 97.5 103.5) (width 0.2) (layer "B.Cu") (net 9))
 (segment (start 103.425 98.56) (end 99.94 98.56) (width 0.2) (layer "F.Cu") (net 10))
 (segment (start 99.94 98.56) (end 97 101.5) (width 0.2) (layer "F.Cu") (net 10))
 (segment (start 97 101.5) (end 96.82 101.32) (width 0.2) (layer "F.Cu") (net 10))
 (segment (start 96.82 101.32) (end 94.54 101.32) (width 0.2) (layer "F.Cu") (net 10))
 (segment (start 100 101) (end 100 103) (width 0.2) (layer "F.Cu") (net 11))
 (segment (start 96.4 106.4) (end 94.54 106.4) (width 0.2) (layer "F.Cu") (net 11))
 (segment (start 103.425 101.1) (end 100.1 101.1) (width 0.2) (layer "F.Cu") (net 11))
 (segment (start 100.1 101.1) (end 100 101) (width 0.2) (layer "F.Cu") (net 11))
 (segment (start 100 103) (end 96.5 106.5) (width 0.2) (layer "F.Cu") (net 11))
 (segment (start 96.5 106.5) (end 96.4 106.4) (width 0.2) (layer "F.Cu") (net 11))
 (segment (start 93.15 127.87) (end 124.37 127.87) (width 0.2) (layer "F.Cu") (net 4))
 (segment (start 124.37 127.87) (end 124.5 128) (width 0.2) (layer "F.Cu") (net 4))
 (segment (start 126.5 120.5) (end 129.5 117.5) (width 0.2) (layer "F.Cu") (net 4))
 (segment (start 129.5 117.5) (end 129.5 95) (width 0.2) (layer "F.Cu") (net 4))
 (segment (start 129.5 95) (end 127.98 93.48) (width 0.2) (layer "F.Cu") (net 4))
 (segment (start 127.98 93.48) (end 126.575 93.48) (width 0.2) (layer "F.Cu") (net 4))
 (segment (start 126.5 126) (end 126.5 120.5) (width 0.2) (layer "F.Cu") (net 4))
 (segment (start 124.5 128) (end 126.5 126) (width 0.2) (layer "F.Cu") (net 4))
 (segment (start 92 126.72) (end 93.15 127.87) (width 0.2) (layer "F.Cu") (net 4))
 (segment (start 88.32 124.18) (end 87.5 125) (width 0.2) (layer "F.Cu") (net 6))
 (segment (start 103.425 88.4) (end 101.1 88.4) (width 0.2) (layer "F.Cu") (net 6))
 (segment (start 101.1 88.4) (end 100 89.5) (width 0.2) (layer "F.Cu") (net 6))
 (segment (start 92 124.18) (end 88.32 124.18) (width 0.2) (layer "F.Cu") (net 6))
 (via (at 87.5 125) (size 0.6) (drill 0.3) (layers "F.Cu" "B.Cu") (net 6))
 (via (at 100 89.5) (size 0.6) (drill 0.3) (layers "F.Cu" "B.Cu") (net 6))
 (segment (start 102 130) (end 99 133) (width 0.2) (layer "B.Cu") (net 6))
 (segment (start 102 126.5) (end 102 130) (width 0.2) (layer "B.Cu") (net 6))
 (segment (start 100 124.5) (end 102 126.5) (width 0.2) (layer "B.Cu") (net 6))
 (segment (start 87 133) (end 87 125.5) (width 0.2) (layer "B.Cu") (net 6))
 (segment (start 99 133) (end 87 133) (width 0.2) (layer "B.Cu") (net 6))
 (segment (start 100 89.5) (end 100 124.5) (width 0.2) (layer "B.Cu") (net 6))
 (segment (start 87 125.5) (end 87.5 125) (width 0.2) (layer "B.Cu") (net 6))
 (segment (start 119.06 98.56) (end 119 98.5) (width 0.2) (layer "F.Cu") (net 2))
 (segment (start 126.575 98.56) (end 119.06 98.56) (width 0.2) (layer "F.Cu") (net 2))
 (segment (start 88 84) (end 88 82.5) (width 0.2) (layer "F.Cu") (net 2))
 (segment (start 92 86.08) (end 90.08 86.08) (width 0.2) (layer "F.Cu") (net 2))
 (segment (start 90.08 86.08) (end 88 84) (width 0.2) (layer "F.Cu") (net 2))
 (via (at 119 98.5) (size 0.6) (drill 0.3) (layers "F.Cu" "B.Cu") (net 2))
 (via (at 88 82.5) (size 0.6) (drill 0.3) (layers "F.Cu" "B.Cu") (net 2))
 (segment (start 88 75.6) (end 88 82.5) (width 0.2) (layer "B.Cu") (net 2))
 (segment (start 119 97.5) (end 118 96.5) (width 0.2) (layer "B.Cu") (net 2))
 (segment (start 117.6 75.6) (end 88 75.6) (width 0.2) (layer "B.Cu") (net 2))
 (segment (start 118 76) (end 117.6 75.6) (width 0.2) (layer "B.Cu") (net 2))
 (segment (start 119 98.5) (end 119 97.5) (width 0.2) (layer "B.Cu") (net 2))
 (segment (start 118 96.5) (end 118 76) (width 0.2) (layer "B.Cu") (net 2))
 (segment (start 134.5329 108.865) (end 133 110.3979) (width 2) (layer "F.Cu") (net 37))
 (segment (start 133 114) (end 135 116) (width 2) (layer "F.Cu") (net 37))
 (segment (start 129 126) (end 130.5 127.5) (width 2) (layer "F.Cu") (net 37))
 (segment (start 129 122) (end 129 126) (width 2) (layer "F.Cu") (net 37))
 (segment (start 135 116) (end 129 122) (width 2) (layer "F.Cu") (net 37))
 (segment (start 133 110.3979) (end 133 114) (width 2) (layer "F.Cu") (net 37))
 (segment (start 129.5 126.5) (end 130.5 127.5) (width 0.2) (layer "F.Cu") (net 37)))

